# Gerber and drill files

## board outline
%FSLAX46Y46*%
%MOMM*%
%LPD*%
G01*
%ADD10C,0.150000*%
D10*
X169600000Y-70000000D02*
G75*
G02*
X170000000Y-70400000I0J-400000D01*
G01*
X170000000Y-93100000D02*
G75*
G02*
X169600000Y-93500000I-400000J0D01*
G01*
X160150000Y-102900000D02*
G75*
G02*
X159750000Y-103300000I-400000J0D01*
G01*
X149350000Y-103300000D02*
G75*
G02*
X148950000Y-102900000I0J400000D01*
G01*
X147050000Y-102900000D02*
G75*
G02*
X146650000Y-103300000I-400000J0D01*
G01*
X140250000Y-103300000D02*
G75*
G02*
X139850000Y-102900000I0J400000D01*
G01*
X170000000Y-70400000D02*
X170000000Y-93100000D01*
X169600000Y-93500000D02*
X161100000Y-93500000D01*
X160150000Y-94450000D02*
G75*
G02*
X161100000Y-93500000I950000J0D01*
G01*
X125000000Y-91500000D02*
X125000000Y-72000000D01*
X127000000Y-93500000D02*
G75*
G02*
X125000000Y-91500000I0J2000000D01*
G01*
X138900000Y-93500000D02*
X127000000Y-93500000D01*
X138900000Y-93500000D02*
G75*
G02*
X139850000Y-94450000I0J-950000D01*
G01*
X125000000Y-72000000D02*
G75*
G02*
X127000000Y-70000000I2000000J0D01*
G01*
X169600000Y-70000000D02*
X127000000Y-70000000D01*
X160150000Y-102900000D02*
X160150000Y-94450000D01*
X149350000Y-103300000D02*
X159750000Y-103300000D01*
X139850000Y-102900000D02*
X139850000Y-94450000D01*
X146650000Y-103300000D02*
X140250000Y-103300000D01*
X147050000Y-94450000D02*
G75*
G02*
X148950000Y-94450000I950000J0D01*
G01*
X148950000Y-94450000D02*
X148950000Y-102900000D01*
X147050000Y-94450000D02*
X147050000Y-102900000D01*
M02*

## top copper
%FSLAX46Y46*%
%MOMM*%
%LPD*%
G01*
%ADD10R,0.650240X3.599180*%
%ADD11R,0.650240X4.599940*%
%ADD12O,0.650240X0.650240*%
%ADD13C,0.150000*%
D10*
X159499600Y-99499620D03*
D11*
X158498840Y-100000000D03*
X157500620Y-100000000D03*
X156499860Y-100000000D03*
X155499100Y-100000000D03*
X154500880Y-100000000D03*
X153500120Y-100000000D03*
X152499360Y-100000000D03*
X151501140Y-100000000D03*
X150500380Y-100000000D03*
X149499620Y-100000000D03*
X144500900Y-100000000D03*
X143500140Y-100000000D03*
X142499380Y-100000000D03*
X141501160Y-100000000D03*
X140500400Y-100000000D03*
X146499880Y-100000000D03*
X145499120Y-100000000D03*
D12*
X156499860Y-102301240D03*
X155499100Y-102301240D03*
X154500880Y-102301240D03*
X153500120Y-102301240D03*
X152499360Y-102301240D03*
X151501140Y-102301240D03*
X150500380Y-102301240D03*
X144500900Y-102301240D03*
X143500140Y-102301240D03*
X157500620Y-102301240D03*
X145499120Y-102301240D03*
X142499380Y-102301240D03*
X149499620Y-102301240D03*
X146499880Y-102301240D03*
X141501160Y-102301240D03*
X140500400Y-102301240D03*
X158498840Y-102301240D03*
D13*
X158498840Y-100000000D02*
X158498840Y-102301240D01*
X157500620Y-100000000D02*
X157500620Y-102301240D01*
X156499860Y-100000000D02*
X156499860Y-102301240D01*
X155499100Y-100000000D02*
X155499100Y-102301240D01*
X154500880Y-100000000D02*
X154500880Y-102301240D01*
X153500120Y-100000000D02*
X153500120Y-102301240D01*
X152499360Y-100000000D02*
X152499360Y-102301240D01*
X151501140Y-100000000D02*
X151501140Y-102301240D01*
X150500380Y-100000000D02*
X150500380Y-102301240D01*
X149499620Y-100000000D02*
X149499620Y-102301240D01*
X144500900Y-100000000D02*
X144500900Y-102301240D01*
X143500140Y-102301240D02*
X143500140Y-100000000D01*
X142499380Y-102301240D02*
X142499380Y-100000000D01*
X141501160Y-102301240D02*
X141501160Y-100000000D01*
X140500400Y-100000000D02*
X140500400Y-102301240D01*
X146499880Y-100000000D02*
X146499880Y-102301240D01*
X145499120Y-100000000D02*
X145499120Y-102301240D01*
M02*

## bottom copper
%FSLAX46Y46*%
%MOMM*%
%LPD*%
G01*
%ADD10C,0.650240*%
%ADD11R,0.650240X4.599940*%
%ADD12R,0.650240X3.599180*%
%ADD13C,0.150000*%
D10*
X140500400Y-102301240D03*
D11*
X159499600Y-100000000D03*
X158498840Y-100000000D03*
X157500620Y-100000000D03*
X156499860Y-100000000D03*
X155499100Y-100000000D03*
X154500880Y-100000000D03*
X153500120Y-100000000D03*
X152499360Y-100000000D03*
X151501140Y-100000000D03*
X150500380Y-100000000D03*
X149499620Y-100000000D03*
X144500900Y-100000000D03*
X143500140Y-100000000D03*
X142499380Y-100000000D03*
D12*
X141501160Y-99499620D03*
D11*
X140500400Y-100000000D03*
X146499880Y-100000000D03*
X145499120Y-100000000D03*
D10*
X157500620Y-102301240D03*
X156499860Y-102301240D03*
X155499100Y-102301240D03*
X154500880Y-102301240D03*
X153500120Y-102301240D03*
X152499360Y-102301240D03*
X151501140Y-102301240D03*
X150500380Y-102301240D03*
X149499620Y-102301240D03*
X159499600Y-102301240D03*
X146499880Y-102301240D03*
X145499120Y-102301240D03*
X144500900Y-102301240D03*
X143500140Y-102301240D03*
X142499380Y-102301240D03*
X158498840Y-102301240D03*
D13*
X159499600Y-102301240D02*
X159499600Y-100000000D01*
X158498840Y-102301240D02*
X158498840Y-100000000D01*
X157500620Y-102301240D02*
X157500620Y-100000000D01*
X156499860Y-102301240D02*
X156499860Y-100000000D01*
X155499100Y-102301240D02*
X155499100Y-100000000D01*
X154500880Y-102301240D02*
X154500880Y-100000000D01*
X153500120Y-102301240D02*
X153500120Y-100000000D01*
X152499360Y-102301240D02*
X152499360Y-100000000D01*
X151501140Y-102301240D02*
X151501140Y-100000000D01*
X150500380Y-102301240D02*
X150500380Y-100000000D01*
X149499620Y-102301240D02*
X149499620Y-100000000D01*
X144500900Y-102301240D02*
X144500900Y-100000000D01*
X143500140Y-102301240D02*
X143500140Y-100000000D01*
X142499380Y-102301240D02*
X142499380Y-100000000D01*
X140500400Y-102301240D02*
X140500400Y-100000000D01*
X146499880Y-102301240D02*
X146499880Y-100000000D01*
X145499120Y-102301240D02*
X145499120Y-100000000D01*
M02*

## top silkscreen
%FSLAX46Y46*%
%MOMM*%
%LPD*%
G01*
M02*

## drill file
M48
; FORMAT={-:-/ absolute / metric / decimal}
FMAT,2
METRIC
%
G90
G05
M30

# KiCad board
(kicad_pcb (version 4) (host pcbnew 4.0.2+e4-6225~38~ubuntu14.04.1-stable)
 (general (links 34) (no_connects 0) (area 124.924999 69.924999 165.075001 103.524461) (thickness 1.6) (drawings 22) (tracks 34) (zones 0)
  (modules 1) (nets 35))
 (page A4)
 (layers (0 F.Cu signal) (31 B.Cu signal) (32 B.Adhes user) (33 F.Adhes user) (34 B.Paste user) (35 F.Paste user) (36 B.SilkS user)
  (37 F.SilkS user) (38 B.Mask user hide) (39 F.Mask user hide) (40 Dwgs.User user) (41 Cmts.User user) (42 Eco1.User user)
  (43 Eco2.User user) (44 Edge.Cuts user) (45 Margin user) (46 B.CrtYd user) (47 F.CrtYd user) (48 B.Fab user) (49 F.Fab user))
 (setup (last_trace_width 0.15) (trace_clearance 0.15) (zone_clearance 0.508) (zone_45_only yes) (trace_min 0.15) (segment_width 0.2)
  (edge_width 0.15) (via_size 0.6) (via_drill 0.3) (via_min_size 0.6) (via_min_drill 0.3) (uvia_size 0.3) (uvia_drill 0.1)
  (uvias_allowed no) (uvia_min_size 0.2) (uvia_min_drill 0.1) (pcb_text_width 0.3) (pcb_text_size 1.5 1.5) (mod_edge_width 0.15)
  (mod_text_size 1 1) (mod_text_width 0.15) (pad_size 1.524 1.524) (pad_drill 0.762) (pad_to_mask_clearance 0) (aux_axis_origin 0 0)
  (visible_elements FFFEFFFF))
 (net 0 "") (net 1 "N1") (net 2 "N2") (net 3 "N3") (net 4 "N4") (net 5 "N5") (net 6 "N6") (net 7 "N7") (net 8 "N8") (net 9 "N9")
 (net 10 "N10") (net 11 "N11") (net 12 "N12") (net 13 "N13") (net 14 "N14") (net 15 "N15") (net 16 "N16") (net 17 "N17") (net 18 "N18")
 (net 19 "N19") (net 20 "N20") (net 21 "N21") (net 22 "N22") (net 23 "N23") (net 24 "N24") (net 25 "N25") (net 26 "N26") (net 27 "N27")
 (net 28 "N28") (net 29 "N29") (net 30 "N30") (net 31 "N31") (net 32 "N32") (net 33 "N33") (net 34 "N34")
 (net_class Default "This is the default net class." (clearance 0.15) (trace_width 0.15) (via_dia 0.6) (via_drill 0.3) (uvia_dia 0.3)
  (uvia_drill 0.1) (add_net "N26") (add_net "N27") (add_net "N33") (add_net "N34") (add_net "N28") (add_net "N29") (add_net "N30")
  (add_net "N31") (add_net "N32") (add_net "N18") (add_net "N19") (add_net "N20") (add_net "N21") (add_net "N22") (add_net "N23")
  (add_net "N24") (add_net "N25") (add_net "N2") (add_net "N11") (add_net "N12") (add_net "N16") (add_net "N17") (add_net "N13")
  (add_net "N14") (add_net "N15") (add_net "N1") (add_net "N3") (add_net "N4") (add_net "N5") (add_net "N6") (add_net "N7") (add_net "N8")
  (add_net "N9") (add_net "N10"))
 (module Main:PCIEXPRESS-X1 (layer B.Cu) (at 150 100 180)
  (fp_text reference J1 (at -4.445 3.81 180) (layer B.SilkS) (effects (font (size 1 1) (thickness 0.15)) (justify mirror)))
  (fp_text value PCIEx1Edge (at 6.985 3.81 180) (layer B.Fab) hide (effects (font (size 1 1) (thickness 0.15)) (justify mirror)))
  (pad B18 connect circle (at 9.4996 -2.30124 180) (size 0.65024 0.65024) (layers B.Cu B.Mask) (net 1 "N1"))
  (pad B1 connect rect (at -9.4996 0 180) (size 0.65024 4.59994) (layers B.Cu B.Mask) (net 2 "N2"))
  (pad B2 connect rect (at -8.49884 0 180) (size 0.65024 4.59994) (layers B.Cu B.Mask) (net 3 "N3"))
  (pad B3 connect rect (at -7.50062 0 180) (size 0.65024 4.59994) (layers B.Cu B.Mask) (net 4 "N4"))
  (pad B4 connect rect (at -6.49986 0 180) (size 0.65024 4.59994) (layers B.Cu B.Mask) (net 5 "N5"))
  (pad B5 connect rect (at -5.4991 0 180) (size 0.65024 4.59994) (layers B.Cu B.Mask) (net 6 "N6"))
  (pad B6 connect rect (at -4.50088 0 180) (size 0.65024 4.59994) (layers B.Cu B.Mask) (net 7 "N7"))
  (pad B7 connect rect (at -3.50012 0 180) (size 0.65024 4.59994) (layers B.Cu B.Mask) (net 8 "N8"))
  (pad B8 connect rect (at -2.49936 0 180) (size 0.65024 4.59994) (layers B.Cu B.Mask) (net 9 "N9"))
  (pad B9 connect rect (at -1.50114 0 180) (size 0.65024 4.59994) (layers B.Cu B.Mask) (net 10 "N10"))
  (pad B10 connect rect (at -0.50038 0 180) (size 0.65024 4.59994) (layers B.Cu B.Mask) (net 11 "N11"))
  (pad B11 connect rect (at 0.50038 0 180) (size 0.65024 4.59994) (layers B.Cu B.Mask) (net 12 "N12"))
  (pad B14 connect rect (at 5.4991 0 180) (size 0.65024 4.59994) (layers B.Cu B.Mask) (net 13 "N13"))
  (pad B15 connect rect (at 6.49986 0 180) (size 0.65024 4.59994) (layers B.Cu B.Mask) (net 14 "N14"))
  (pad B16 connect rect (at 7.50062 0 180) (size 0.65024 4.59994) (layers B.Cu B.Mask) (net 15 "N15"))
  (pad B17 connect rect (at 8.49884 0.50038 180) (size 0.65024 3.59918) (layers B.Cu B.Mask))
  (pad B18 connect rect (at 9.4996 0 180) (size 0.65024 4.59994) (layers B.Cu B.Mask) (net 1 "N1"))
  (pad B12 connect rect (at 3.50012 0 180) (size 0.65024 4.59994) (layers B.Cu B.Mask) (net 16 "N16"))
  (pad B13 connect rect (at 4.50088 0 180) (size 0.65024 4.59994) (layers B.Cu B.Mask) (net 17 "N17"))
  (pad A1 connect rect (at -9.4996 0.50038 180) (size 0.65024 3.59918) (layers F.Cu F.Mask))
  (pad A2 connect rect (at -8.49884 0 180) (size 0.65024 4.59994) (layers F.Cu F.Mask) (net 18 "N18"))
  (pad A3 connect rect (at -7.50062 0 180) (size 0.65024 4.59994) (layers F.Cu F.Mask) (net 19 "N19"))
  (pad A4 connect rect (at -6.49986 0 180) (size 0.65024 4.59994) (layers F.Cu F.Mask) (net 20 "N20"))
  (pad A5 connect rect (at -5.4991 0 180) (size 0.65024 4.59994) (layers F.Cu F.Mask) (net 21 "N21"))
  (pad A6 connect rect (at -4.50088 0 180) (size 0.65024 4.59994) (layers F.Cu F.Mask) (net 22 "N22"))
  (pad A7 connect rect (at -3.50012 0 180) (size 0.65024 4.59994) (layers F.Cu F.Mask) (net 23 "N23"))
  (pad A8 connect rect (at -2.49936 0 180) (size 0.65024 4.59994) (layers F.Cu F.Mask) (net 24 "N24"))
  (pad A9 connect rect (at -1.50114 0 180) (size 0.65024 4.59994) (layers F.Cu F.Mask) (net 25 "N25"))
  (pad A10 connect rect (at -0.50038 0 180) (size 0.65024 4.59994) (layers F.Cu F.Mask) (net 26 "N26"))
  (pad A11 connect rect (at 0.50038 0 180) (size 0.65024 4.59994) (layers F.Cu F.Mask) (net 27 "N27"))
  (pad A14 connect rect (at 5.4991 0 180) (size 0.65024 4.59994) (layers F.Cu F.Mask) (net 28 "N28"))
  (pad A15 connect rect (at 6.49986 0 180) (size 0.65024 4.59994) (layers F.Cu F.Mask) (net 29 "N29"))
  (pad A16 connect rect (at 7.50062 0 180) (size 0.65024 4.59994) (layers F.Cu F.Mask) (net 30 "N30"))
  (pad A17 connect rect (at 8.49884 0 180) (size 0.65024 4.59994) (layers F.Cu F.Mask) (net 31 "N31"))
  (pad A18 connect rect (at 9.4996 0 180) (size 0.65024 4.59994) (layers F.Cu F.Mask) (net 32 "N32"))
  (pad A12 connect rect (at 3.50012 0 180) (size 0.65024 4.59994) (layers F.Cu F.Mask) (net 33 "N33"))
  (pad A13 connect rect (at 4.50088 0 180) (size 0.65024 4.59994) (layers F.Cu F.Mask) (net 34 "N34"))
  (pad B3 connect circle (at -7.50062 -2.30124 180) (size 0.65024 0.65024) (layers B.Cu B.Mask) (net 4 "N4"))
  (pad B4 connect circle (at -6.49986 -2.30124 180) (size 0.65024 0.65024) (layers B.Cu B.Mask) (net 5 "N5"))
  (pad B5 connect circle (at -5.4991 -2.30124 180) (size 0.65024 0.65024) (layers B.Cu B.Mask) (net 6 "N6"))
  (pad B6 connect circle (at -4.50088 -2.30124 180) (size 0.65024 0.65024) (layers B.Cu B.Mask) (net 7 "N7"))
  (pad B7 connect circle (at -3.50012 -2.30124 180) (size 0.65024 0.65024) (layers B.Cu B.Mask) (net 8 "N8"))
  (pad B8 connect circle (at -2.49936 -2.30124 180) (size 0.65024 0.65024) (layers B.Cu B.Mask) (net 9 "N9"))
  (pad B9 connect circle (at -1.50114 -2.30124 180) (size 0.65024 0.65024) (layers B.Cu B.Mask) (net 10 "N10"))
  (pad B10 connect circle (at -0.50038 -2.30124 180) (size 0.65024 0.65024) (layers B.Cu B.Mask) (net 11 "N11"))
  (pad B11 connect circle (at 0.50038 -2.30124 180) (size 0.65024 0.65024) (layers B.Cu B.Mask) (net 12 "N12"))
  (pad B1 connect circle (at -9.4996 -2.30124 180) (size 0.65024 0.65024) (layers B.Cu B.Mask) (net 2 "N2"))
  (pad B12 connect circle (at 3.50012 -2.30124 180) (size 0.65024 0.65024) (layers B.Cu B.Mask) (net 16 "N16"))
  (pad B13 connect circle (at 4.50088 -2.30124 180) (size 0.65024 0.65024) (layers B.Cu B.Mask) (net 17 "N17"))
  (pad B14 connect circle (at 5.4991 -2.30124 180) (size 0.65024 0.65024) (layers B.Cu B.Mask) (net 13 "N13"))
  (pad B15 connect circle (at 6.49986 -2.30124 180) (size 0.65024 0.65024) (layers B.Cu B.Mask) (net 14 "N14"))
  (pad B16 connect circle (at 7.50062 -2.30124 180) (size 0.65024 0.65024) (layers B.Cu B.Mask) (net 15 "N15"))
  (pad B2 connect circle (at -8.49884 -2.30124 180) (size 0.65024 0.65024) (layers B.Cu B.Mask) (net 3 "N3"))
  (pad A4 connect oval (at -6.49986 -2.30124 90) (size 0.65024 0.65024) (layers F.Cu F.Mask) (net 20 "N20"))
  (pad A5 connect oval (at -5.4991 -2.30124 90) (size 0.65024 0.65024) (layers F.Cu F.Mask) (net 21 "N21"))
  (pad A6 connect oval (at -4.50088 -2.30124 90) (size 0.65024 0.65024) (layers F.Cu F.Mask) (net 22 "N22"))
  (pad A7 connect oval (at -3.50012 -2.30124 90) (size 0.65024 0.65024) (layers F.Cu F.Mask) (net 23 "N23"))
  (pad A8 connect oval (at -2.49936 -2.30124 90) (size 0.65024 0.65024) (layers F.Cu F.Mask) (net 24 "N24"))
  (pad A9 connect oval (at -1.50114 -2.30124 90) (size 0.65024 0.65024) (layers F.Cu F.Mask) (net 25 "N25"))
  (pad A10 connect oval (at -0.50038 -2.30124 90) (size 0.65024 0.65024) (layers F.Cu F.Mask) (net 26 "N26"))
  (pad A14 connect oval (at 5.4991 -2.30124 90) (size 0.65024 0.65024) (layers F.Cu F.Mask) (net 28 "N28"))
  (pad A15 connect oval (at 6.49986 -2.30124 90) (size 0.65024 0.65024) (layers F.Cu F.Mask) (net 29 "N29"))
  (pad A3 connect oval (at -7.50062 -2.30124 90) (size 0.65024 0.65024) (layers F.Cu F.Mask) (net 19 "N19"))
  (pad A13 connect oval (at 4.50088 -2.30124 90) (size 0.65024 0.65024) (layers F.Cu F.Mask) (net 34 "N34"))
  (pad A16 connect oval (at 7.50062 -2.30124 90) (size 0.65024 0.65024) (layers F.Cu F.Mask) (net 30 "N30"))
  (pad A11 connect oval (at 0.50038 -2.30124 90) (size 0.65024 0.65024) (layers F.Cu F.Mask) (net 27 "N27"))
  (pad A12 connect oval (at 3.50012 -2.30124 90) (size 0.65024 0.65024) (layers F.Cu F.Mask) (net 33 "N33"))
  (pad A17 connect oval (at 8.49884 -2.30124 90) (size 0.65024 0.65024) (layers F.Cu F.Mask) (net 31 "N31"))
  (pad A18 connect oval (at 9.4996 -2.30124 90) (size 0.65024 0.65024) (layers F.Cu F.Mask) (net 32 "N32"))
  (pad A2 connect oval (at -8.49884 -2.30124 90) (size 0.65024 0.65024) (layers F.Cu F.Mask) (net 18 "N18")))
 (gr_arc (start 169.6 70.4) (end 170 70.4) (angle -90) (layer Edge.Cuts) (width 0.15))
 (gr_arc (start 169.6 93.1) (end 169.6 93.5) (angle -90) (layer Edge.Cuts) (width 0.15))
 (gr_arc (start 159.75 102.9) (end 160.15 102.9) (angle 90) (layer Edge.Cuts) (width 0.15))
 (gr_arc (start 149.35 102.9) (end 148.95 102.9) (angle -90) (layer Edge.Cuts) (width 0.15))
 (gr_arc (start 146.65 102.9) (end 147.05 102.9) (angle 90) (layer Edge.Cuts) (width 0.15))
 (gr_arc (start 140.25 102.9) (end 139.85 102.9) (angle -90) (layer Edge.Cuts) (width 0.15))
 (gr_line (start 170 70.4) (end 170 93.1) (angle 90) (layer Edge.Cuts) (width 0.15))
 (gr_line (start 169.6 93.5) (end 161.1 93.5) (angle 90) (layer Edge.Cuts) (width 0.15))
 (gr_arc (start 161.1 94.45) (end 160.15 94.45) (angle 90) (layer Edge.Cuts) (width 0.15))
 (gr_line (start 125 91.5) (end 125 72) (angle 90) (layer Edge.Cuts) (width 0.15))
 (gr_arc (start 127 91.5) (end 127 93.5) (angle 90) (layer Edge.Cuts) (width 0.15))
 (gr_line (start 138.9 93.5) (end 127 93.5) (angle 90) (layer Edge.Cuts) (width 0.15))
 (gr_arc (start 138.9 94.45) (end 139.85 94.45) (angle -90) (layer Edge.Cuts) (width 0.15))
 (gr_arc (start 127 72) (end 125 72) (angle 90) (layer Edge.Cuts) (width 0.15))
 (gr_line (start 169.6 70) (end 127 70) (angle 90) (layer Edge.Cuts) (width 0.15))
 (gr_line (start 160.15 102.9) (end 160.15 94.45) (angle 90) (layer Edge.Cuts) (width 0.15))
 (gr_line (start 149.35 103.3) (end 159.75 103.3) (angle 90) (layer Edge.Cuts) (width 0.15))
 (gr_line (start 139.85 102.9) (end 139.85 94.45) (angle 90) (layer Edge.Cuts) (width 0.15))
 (gr_line (start 146.65 103.3) (end 140.25 103.3) (angle 90) (layer Edge.Cuts) (width 0.15))
 (gr_arc (start 148 94.45) (end 147.05 94.45) (angle 180) (layer Edge.Cuts) (width 0.15))
 (gr_line (start 148.95 94.45) (end 148.95 102.9) (angle 90) (layer Edge.Cuts) (width 0.15))
 (gr_line (start 147.05 94.45) (end 147.05 102.9) (angle 90) (layer Edge.Cuts) (width 0.15))
 (segment (start 159.4996 102.30124) (end 159.4996 100) (width 0.15) (layer B.Cu) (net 2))
 (segment (start 158.49884 102.30124) (end 158.49884 100) (width 0.15) (layer B.Cu) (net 3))
 (segment (start 157.50062 102.30124) (end 157.50062 100) (width 0.15) (layer B.Cu) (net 4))
 (segment (start 156.49986 102.30124) (end 156.49986 100) (width 0.15) (layer B.Cu) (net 5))
 (segment (start 155.4991 102.30124) (end 155.4991 100) (width 0.15) (layer B.Cu) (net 6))
 (segment (start 154.50088 102.30124) (end 154.50088 100) (width 0.15) (layer B.Cu) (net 7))
 (segment (start 153.50012 102.30124) (end 153.50012 100) (width 0.15) (layer B.Cu) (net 8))
 (segment (start 152.49936 102.30124) (end 152.49936 100) (width 0.15) (layer B.Cu) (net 9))
 (segment (start 151.50114 102.30124) (end 151.50114 100) (width 0.15) (layer B.Cu) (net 10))
 (segment (start 150.50038 102.30124) (end 150.50038 100) (width 0.15) (layer B.Cu) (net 11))
 (segment (start 149.49962 102.30124) (end 149.49962 100) (width 0.15) (layer B.Cu) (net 12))
 (segment (start 144.5009 102.30124) (end 144.5009 100) (width 0.15) (layer B.Cu) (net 13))
 (segment (start 143.50014 102.30124) (end 143.50014 100) (width 0.15) (layer B.Cu) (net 14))
 (segment (start 142.49938 102.30124) (end 142.49938 100) (width 0.15) (layer B.Cu) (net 15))
 (segment (start 140.5004 102.30124) (end 140.5004 100) (width 0.15) (layer B.Cu) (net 1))
 (segment (start 146.49988 102.30124) (end 146.49988 100) (width 0.15) (layer B.Cu) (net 16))
 (segment (start 145.49912 102.30124) (end 145.49912 100) (width 0.15) (layer B.Cu) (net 17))
 (segment (start 158.49884 100) (end 158.49884 102.30124) (width 0.15) (layer F.Cu) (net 18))
 (segment (start 157.50062 100) (end 157.50062 102.30124) (width 0.15) (layer F.Cu) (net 19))
 (segment (start 156.49986 100) (end 156.49986 102.30124) (width 0.15) (layer F.Cu) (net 20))
 (segment (start 155.4991 100) (end 155.4991 102.30124) (width 0.15) (layer F.Cu) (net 21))
 (segment (start 154.50088 100) (end 154.50088 102.30124) (width 0.15) (layer F.Cu) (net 22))
 (segment (start 153.50012 100) (end 153.50012 102.30124) (width 0.15) (layer F.Cu) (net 23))
 (segment (start 152.49936 100) (end 152.49936 102.30124) (width 0.15) (layer F.Cu) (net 24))
 (segment (start 151.50114 100) (end 151.50114 102.30124) (width 0.15) (layer F.Cu) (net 25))
 (segment (start 150.50038 100) (end 150.50038 102.30124) (width 0.15) (layer F.Cu) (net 26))
 (segment (start 149.49962 100) (end 149.49962 102.30124) (width 0.15) (layer F.Cu) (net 27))
 (segment (start 144.5009 100) (end 144.5009 102.30124) (width 0.15) (layer F.Cu) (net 28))
 (segment (start 143.50014 102.30124) (end 143.50014 100) (width 0.15) (layer F.Cu) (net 29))
 (segment (start 142.49938 102.30124) (end 142.49938 100) (width 0.15) (layer F.Cu) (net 30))
 (segment (start 141.50116 102.30124) (end 141.50116 100) (width 0.15) (layer F.Cu) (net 31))
 (segment (start 140.5004 100) (end 140.5004 102.30124) (width 0.15) (layer F.Cu) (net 32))
 (segment (start 146.49988 100) (end 146.49988 102.30124) (width 0.15) (layer F.Cu) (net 33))
 (segment (start 145.49912 100) (end 145.49912 102.30124) (width 0.15) (layer F.Cu) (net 34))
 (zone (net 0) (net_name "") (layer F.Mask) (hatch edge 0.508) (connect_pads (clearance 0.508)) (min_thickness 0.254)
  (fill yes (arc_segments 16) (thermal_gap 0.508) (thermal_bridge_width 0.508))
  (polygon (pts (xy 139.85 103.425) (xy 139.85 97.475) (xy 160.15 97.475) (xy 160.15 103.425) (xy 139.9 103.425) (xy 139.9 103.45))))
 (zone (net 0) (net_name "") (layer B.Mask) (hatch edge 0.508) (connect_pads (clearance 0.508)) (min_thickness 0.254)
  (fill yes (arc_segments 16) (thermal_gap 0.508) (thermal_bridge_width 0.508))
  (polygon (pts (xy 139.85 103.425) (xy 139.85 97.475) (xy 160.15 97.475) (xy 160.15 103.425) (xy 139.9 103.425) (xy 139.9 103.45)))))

